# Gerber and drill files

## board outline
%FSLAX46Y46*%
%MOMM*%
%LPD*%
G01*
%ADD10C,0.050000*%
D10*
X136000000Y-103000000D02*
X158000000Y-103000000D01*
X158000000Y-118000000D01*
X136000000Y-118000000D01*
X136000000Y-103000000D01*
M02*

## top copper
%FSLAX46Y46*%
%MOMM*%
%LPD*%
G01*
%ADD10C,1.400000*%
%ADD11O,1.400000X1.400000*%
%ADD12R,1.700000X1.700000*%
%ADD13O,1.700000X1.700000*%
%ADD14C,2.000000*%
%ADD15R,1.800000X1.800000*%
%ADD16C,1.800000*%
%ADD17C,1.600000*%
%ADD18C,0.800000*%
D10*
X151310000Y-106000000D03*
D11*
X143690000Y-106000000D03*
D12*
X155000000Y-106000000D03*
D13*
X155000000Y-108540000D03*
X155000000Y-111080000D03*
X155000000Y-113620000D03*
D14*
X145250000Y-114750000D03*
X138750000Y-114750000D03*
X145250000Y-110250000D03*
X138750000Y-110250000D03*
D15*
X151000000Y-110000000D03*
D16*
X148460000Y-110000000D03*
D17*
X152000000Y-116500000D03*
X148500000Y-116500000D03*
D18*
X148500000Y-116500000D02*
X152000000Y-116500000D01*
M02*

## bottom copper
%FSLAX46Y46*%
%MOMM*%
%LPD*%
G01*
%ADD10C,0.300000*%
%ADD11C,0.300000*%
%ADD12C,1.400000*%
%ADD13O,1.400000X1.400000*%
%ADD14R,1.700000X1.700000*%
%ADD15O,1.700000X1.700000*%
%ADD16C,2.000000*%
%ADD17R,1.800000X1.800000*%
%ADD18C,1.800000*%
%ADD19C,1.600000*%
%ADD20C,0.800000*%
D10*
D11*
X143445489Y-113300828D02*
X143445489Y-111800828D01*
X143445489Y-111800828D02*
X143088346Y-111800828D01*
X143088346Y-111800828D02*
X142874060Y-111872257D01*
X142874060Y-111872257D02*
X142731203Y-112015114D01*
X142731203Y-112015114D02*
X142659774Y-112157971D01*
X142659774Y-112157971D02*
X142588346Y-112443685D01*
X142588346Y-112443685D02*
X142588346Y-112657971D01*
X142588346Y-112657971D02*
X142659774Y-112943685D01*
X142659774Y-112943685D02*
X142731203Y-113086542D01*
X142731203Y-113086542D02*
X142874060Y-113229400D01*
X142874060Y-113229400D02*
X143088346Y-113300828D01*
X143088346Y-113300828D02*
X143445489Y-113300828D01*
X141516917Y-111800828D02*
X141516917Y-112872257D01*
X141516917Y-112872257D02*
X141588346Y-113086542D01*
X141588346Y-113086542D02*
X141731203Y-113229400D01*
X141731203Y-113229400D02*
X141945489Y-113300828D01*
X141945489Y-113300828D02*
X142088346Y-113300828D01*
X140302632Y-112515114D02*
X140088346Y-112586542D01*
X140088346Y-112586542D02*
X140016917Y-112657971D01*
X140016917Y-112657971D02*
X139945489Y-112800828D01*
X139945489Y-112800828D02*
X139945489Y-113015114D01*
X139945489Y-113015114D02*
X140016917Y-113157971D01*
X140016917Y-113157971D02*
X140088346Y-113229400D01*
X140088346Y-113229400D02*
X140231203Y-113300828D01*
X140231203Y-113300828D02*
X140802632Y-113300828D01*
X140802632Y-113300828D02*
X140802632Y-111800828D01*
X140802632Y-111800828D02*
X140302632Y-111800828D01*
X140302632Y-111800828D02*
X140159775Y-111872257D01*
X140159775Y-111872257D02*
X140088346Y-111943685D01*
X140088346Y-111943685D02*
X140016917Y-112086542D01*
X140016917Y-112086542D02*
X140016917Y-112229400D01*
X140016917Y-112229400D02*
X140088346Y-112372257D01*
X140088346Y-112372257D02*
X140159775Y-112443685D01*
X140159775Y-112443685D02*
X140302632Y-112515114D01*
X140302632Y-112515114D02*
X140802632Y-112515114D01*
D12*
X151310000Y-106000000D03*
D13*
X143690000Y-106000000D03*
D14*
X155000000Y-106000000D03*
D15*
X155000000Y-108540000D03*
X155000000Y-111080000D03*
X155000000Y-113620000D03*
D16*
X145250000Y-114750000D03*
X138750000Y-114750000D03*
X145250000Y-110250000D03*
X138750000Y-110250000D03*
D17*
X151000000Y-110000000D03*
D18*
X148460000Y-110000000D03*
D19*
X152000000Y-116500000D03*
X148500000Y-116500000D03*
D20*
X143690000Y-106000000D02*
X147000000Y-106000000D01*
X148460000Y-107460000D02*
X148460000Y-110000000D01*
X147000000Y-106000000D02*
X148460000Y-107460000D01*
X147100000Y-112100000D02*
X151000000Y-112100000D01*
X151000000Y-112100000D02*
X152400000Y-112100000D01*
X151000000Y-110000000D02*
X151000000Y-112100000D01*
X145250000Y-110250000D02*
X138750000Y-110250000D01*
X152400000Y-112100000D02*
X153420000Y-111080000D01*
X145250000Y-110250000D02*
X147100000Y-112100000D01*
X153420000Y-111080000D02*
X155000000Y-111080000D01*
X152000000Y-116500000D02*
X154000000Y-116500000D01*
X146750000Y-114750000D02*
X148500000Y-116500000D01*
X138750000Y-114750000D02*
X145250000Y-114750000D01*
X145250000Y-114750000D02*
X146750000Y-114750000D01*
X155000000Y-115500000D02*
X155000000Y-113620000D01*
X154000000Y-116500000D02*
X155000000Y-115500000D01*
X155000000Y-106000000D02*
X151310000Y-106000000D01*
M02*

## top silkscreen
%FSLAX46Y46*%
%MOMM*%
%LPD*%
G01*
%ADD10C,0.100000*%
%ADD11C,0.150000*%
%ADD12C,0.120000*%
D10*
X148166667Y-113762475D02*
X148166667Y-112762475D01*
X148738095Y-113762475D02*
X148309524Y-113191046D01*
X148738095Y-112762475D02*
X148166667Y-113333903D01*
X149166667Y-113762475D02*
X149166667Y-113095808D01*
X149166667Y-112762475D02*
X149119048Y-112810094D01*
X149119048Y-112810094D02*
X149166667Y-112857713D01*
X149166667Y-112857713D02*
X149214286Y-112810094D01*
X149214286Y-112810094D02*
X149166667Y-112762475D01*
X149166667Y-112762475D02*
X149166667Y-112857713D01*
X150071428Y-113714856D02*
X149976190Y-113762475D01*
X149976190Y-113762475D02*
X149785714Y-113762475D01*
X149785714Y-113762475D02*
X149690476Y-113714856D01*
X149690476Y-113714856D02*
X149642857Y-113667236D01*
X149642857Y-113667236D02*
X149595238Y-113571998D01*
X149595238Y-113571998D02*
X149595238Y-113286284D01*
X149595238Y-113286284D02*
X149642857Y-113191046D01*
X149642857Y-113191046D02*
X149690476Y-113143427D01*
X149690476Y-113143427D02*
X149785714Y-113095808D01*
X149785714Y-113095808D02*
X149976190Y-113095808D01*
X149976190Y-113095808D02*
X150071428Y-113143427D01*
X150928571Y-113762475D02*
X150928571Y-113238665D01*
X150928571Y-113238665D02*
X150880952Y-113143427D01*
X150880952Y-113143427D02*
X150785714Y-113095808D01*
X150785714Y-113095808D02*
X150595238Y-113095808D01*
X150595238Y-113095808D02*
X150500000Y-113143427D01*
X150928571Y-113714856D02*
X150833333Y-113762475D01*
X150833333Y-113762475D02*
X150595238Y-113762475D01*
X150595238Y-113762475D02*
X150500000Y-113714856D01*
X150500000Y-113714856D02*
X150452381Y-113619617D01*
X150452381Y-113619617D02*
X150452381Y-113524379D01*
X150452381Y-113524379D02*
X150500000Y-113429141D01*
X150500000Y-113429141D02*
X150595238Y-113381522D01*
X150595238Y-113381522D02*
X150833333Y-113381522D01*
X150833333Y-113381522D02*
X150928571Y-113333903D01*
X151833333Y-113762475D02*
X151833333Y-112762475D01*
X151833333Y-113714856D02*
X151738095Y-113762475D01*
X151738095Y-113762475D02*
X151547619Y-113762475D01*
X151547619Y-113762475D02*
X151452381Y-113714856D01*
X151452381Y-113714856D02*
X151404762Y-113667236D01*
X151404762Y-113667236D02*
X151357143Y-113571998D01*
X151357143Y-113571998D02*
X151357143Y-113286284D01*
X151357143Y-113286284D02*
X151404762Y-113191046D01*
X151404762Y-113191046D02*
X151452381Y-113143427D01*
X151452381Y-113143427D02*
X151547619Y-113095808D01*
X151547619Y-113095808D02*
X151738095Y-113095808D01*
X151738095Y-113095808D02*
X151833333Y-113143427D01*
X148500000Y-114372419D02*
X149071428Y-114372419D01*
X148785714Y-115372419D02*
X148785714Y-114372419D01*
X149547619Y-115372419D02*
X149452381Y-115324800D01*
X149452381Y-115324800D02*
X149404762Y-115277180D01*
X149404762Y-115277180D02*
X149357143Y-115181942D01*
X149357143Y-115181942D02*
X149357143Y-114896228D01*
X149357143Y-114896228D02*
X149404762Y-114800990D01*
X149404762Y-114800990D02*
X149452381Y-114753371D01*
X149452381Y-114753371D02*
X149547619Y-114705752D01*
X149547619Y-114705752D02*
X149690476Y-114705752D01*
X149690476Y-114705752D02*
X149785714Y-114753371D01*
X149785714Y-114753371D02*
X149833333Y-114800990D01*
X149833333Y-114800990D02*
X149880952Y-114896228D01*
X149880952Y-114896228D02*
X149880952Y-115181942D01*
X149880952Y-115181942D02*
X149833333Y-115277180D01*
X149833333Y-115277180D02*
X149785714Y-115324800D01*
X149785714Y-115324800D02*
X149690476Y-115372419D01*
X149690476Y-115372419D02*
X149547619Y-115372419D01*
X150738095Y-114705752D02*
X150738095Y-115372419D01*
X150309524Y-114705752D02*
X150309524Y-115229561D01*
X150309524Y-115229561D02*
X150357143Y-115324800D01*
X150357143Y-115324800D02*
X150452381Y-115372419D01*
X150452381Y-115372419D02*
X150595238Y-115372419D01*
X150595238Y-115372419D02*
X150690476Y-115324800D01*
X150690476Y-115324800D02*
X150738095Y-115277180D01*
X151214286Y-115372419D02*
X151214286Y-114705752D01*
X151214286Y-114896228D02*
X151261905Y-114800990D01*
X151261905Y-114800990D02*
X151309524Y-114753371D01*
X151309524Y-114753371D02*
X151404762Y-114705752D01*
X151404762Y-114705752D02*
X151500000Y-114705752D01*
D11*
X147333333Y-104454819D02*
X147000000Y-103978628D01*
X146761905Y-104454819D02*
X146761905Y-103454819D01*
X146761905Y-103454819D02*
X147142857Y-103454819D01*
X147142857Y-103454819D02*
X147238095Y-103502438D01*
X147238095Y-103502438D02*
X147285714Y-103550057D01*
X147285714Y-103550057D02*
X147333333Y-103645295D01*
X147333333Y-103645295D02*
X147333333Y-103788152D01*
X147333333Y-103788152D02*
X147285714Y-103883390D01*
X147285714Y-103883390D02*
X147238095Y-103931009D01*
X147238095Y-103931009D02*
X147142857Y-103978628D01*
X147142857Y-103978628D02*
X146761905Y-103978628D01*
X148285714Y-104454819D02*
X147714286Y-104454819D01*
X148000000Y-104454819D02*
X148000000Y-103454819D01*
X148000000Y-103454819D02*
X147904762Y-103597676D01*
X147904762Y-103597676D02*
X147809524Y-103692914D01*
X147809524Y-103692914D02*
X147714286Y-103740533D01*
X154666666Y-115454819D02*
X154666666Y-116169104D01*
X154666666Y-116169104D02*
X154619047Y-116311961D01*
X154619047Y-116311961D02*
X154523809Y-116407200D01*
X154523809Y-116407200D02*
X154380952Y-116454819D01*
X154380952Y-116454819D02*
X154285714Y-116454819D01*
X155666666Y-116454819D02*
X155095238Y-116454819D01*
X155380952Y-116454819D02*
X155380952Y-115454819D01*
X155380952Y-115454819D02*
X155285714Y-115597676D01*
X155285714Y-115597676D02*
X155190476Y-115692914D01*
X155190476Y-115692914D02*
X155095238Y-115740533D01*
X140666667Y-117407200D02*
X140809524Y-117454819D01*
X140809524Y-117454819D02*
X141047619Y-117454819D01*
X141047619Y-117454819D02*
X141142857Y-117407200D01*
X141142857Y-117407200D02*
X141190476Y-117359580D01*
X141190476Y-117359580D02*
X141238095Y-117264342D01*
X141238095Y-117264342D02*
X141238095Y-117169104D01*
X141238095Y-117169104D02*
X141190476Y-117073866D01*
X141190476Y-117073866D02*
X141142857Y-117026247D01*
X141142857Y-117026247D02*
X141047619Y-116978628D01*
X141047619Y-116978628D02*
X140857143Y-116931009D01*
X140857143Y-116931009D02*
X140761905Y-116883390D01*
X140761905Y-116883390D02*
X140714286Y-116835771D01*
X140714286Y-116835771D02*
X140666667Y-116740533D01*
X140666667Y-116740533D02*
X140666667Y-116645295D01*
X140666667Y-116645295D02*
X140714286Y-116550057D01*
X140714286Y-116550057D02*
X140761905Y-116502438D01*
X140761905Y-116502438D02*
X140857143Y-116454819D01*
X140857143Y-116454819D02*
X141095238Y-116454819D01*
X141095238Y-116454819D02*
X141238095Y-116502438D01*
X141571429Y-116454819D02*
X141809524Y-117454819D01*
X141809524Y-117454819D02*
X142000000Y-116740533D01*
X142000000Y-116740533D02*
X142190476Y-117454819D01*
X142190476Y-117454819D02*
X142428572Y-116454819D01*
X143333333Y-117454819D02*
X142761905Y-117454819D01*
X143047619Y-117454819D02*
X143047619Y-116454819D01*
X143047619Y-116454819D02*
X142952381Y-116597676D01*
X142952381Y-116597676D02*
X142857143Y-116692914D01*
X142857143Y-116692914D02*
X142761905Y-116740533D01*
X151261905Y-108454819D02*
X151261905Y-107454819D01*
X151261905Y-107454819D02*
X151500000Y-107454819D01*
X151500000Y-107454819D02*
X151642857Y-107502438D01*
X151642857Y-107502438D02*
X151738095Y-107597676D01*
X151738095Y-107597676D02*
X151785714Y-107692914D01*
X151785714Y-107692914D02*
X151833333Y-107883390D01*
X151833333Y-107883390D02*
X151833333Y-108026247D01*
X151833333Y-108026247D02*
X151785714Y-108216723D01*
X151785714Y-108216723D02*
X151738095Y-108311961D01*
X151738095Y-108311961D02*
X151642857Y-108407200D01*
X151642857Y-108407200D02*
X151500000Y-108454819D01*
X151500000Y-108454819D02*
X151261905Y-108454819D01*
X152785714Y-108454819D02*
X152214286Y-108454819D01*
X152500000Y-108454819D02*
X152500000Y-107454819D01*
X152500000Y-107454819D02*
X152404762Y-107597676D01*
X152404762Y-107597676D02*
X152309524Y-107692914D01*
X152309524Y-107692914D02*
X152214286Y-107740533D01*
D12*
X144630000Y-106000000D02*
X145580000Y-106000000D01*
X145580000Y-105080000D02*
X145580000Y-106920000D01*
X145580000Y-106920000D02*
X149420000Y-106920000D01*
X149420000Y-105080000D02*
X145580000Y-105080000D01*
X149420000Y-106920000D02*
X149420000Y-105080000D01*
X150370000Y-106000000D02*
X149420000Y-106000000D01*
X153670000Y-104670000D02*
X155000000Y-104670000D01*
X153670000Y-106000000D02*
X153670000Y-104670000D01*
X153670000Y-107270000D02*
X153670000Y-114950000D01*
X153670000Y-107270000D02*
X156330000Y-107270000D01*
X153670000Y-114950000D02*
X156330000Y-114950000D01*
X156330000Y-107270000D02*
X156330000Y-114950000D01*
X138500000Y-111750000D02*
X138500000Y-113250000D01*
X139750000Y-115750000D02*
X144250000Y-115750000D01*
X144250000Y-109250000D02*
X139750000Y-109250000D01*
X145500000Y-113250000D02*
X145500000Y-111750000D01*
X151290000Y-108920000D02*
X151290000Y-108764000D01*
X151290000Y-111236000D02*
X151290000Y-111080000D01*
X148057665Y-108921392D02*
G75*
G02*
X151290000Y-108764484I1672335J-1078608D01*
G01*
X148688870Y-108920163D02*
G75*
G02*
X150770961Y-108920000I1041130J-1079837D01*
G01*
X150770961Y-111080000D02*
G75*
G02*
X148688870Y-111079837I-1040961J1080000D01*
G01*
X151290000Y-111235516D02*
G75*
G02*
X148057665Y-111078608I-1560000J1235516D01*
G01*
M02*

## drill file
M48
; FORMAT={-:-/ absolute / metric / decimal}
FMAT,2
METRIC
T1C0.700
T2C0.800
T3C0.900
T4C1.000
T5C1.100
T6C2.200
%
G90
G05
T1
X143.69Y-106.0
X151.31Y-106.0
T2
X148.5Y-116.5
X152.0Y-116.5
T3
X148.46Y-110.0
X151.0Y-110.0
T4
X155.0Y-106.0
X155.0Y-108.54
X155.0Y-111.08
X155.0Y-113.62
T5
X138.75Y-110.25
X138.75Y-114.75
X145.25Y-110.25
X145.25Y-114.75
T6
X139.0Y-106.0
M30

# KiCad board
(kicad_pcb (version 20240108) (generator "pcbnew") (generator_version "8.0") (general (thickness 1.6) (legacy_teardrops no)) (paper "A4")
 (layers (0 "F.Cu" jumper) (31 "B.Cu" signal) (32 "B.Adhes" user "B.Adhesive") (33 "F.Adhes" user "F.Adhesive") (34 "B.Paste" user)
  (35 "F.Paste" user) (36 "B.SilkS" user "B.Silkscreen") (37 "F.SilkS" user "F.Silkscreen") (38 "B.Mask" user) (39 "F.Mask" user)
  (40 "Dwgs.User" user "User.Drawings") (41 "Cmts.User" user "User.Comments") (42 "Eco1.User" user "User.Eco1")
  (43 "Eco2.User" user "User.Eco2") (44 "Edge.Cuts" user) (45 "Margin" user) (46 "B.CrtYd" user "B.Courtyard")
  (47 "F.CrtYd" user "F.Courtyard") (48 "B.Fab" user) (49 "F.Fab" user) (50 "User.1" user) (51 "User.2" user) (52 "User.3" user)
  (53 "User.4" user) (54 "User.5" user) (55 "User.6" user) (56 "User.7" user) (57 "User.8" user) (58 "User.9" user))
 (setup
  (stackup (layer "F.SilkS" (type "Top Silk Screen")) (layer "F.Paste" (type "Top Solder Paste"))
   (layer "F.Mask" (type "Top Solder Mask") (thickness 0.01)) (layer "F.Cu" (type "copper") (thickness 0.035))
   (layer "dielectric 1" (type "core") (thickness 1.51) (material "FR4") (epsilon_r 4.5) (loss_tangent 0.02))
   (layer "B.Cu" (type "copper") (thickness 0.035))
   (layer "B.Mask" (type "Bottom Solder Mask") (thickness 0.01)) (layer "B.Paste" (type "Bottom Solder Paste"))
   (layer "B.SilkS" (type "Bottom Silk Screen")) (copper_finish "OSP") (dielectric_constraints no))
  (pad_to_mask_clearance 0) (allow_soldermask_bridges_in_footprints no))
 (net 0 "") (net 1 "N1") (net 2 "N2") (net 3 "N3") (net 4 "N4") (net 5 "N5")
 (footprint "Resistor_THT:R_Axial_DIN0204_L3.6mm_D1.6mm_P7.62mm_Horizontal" (layer "F.Cu") (at 151.31 106 180)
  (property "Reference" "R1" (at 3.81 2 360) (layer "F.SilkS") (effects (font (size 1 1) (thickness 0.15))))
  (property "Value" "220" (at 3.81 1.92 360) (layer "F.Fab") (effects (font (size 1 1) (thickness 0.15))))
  (fp_line (start 6.68 0) (end 5.73 0) (stroke (width 0.12) (type solid)) (layer "F.SilkS"))
  (fp_line (start 5.73 0.92) (end 5.73 -0.92) (stroke (width 0.12) (type solid)) (layer "F.SilkS"))
  (fp_line (start 5.73 -0.92) (end 1.89 -0.92) (stroke (width 0.12) (type solid)) (layer "F.SilkS"))
  (fp_line (start 1.89 0.92) (end 5.73 0.92) (stroke (width 0.12) (type solid)) (layer "F.SilkS"))
  (fp_line (start 1.89 -0.92) (end 1.89 0.92) (stroke (width 0.12) (type solid)) (layer "F.SilkS"))
  (fp_line (start 0.94 0) (end 1.89 0) (stroke (width 0.12) (type solid)) (layer "F.SilkS"))
  (pad "1" thru_hole circle (at 0 0 180) (size 1.4 1.4) (drill 0.7) (layers "*.Cu" "*.Mask") (remove_unused_layers no) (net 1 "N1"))
  (pad "2" thru_hole oval (at 7.62 0 180) (size 1.4 1.4) (drill 0.7) (layers "*.Cu" "*.Mask") (remove_unused_layers no) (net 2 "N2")))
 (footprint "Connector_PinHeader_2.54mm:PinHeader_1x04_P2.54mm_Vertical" (layer "F.Cu") (at 155 106)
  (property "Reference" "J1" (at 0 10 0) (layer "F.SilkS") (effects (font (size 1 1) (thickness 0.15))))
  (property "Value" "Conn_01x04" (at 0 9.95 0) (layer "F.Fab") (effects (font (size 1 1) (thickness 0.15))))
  (fp_line (start -1.33 -1.33) (end 0 -1.33) (stroke (width 0.12) (type solid)) (layer "F.SilkS"))
  (fp_line (start -1.33 0) (end -1.33 -1.33) (stroke (width 0.12) (type solid)) (layer "F.SilkS"))
  (fp_line (start -1.33 1.27) (end -1.33 8.95) (stroke (width 0.12) (type solid)) (layer "F.SilkS"))
  (fp_line (start -1.33 1.27) (end 1.33 1.27) (stroke (width 0.12) (type solid)) (layer "F.SilkS"))
  (fp_line (start -1.33 8.95) (end 1.33 8.95) (stroke (width 0.12) (type solid)) (layer "F.SilkS"))
  (fp_line (start 1.33 1.27) (end 1.33 8.95) (stroke (width 0.12) (type solid)) (layer "F.SilkS"))
  (pad "1" thru_hole rect (at 0 0) (size 1.7 1.7) (drill 1) (layers "*.Cu" "*.Mask") (remove_unused_layers no) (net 1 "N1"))
  (pad "2" thru_hole oval (at 0 2.54) (size 1.7 1.7) (drill 1) (layers "*.Cu" "*.Mask") (remove_unused_layers no) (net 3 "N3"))
  (pad "3" thru_hole oval (at 0 5.08) (size 1.7 1.7) (drill 1) (layers "*.Cu" "*.Mask") (remove_unused_layers no) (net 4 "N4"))
  (pad "4" thru_hole oval (at 0 7.62) (size 1.7 1.7) (drill 1) (layers "*.Cu" "*.Mask") (remove_unused_layers no) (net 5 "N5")))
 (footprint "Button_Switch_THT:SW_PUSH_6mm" (layer "F.Cu") (at 145.25 114.75 180)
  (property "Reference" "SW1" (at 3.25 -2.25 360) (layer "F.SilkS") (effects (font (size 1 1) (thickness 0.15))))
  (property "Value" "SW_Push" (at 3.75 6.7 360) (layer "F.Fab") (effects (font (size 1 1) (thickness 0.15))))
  (fp_line (start 6.75 3) (end 6.75 1.5) (stroke (width 0.12) (type solid)) (layer "F.SilkS"))
  (fp_line (start 5.5 -1) (end 1 -1) (stroke (width 0.12) (type solid)) (layer "F.SilkS"))
  (fp_line (start 1 5.5) (end 5.5 5.5) (stroke (width 0.12) (type solid)) (layer "F.SilkS"))
  (fp_line (start -0.25 1.5) (end -0.25 3) (stroke (width 0.12) (type solid)) (layer "F.SilkS"))
  (pad "1" thru_hole circle (at 0 0 270) (size 2 2) (drill 1.1) (layers "*.Cu" "*.Mask") (remove_unused_layers no) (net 5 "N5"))
  (pad "1" thru_hole circle (at 6.5 0 270) (size 2 2) (drill 1.1) (layers "*.Cu" "*.Mask") (remove_unused_layers no) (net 5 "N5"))
  (pad "2" thru_hole circle (at 0 4.5 270) (size 2 2) (drill 1.1) (layers "*.Cu" "*.Mask") (remove_unused_layers no) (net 4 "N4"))
  (pad "2" thru_hole circle (at 6.5 4.5 270) (size 2 2) (drill 1.1) (layers "*.Cu" "*.Mask") (remove_unused_layers no) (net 4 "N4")))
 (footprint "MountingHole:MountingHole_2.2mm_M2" (layer "F.Cu") (at 139 106)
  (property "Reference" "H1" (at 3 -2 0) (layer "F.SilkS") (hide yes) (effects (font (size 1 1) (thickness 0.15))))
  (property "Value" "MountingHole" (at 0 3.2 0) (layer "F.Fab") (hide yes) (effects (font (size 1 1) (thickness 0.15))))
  (pad "" np_thru_hole circle (at 0 0) (size 2.2 2.2) (drill 2.2) (layers "*.Cu" "*.Mask")))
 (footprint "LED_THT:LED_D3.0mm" (layer "F.Cu") (at 151 110 180)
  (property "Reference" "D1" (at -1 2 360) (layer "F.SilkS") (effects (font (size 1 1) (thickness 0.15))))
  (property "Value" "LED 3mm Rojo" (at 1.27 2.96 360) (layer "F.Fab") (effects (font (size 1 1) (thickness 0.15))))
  (fp_line (start -0.29 1.08) (end -0.29 1.236) (stroke (width 0.12) (type solid)) (layer "F.SilkS"))
  (fp_line (start -0.29 -1.236) (end -0.29 -1.08) (stroke (width 0.12) (type solid)) (layer "F.SilkS"))
  (fp_arc (start 2.942335 1.078608) (mid 1.366487 1.987659) (end -0.29 1.235516) (stroke (width 0.12) (type solid)) (layer "F.SilkS"))
  (fp_arc (start 2.31113 1.079837) (mid 1.270117 1.5) (end 0.229039 1.08) (stroke (width 0.12) (type solid)) (layer "F.SilkS"))
  (fp_arc (start 0.229039 -1.08) (mid 1.270117 -1.5) (end 2.31113 -1.079837) (stroke (width 0.12) (type solid)) (layer "F.SilkS"))
  (fp_arc (start -0.29 -1.235516) (mid 1.366487 -1.987659) (end 2.942335 -1.078608) (stroke (width 0.12) (type solid)) (layer "F.SilkS"))
  (pad "1" thru_hole rect (at 0 0 180) (size 1.8 1.8) (drill 0.9) (layers "*.Cu" "*.Mask") (remove_unused_layers no) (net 4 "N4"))
  (pad "2" thru_hole circle (at 2.54 0 180) (size 1.8 1.8) (drill 0.9) (layers "*.Cu" "*.Mask") (remove_unused_layers no) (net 2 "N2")))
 (gr_rect (start 136 103) (end 158 118) (stroke (width 0.05) (type default)) (fill none) (layer "Edge.Cuts"))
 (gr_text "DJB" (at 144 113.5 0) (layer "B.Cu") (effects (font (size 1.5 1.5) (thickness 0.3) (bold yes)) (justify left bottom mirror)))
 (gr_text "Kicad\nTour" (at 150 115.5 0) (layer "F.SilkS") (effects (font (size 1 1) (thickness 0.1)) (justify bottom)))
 (segment (start 143.69 106) (end 147 106) (width 0.8) (layer "B.Cu") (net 2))
 (segment (start 148.46 107.46) (end 148.46 110) (width 0.8) (layer "B.Cu") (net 2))
 (segment (start 147 106) (end 148.46 107.46) (width 0.8) (layer "B.Cu") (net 2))
 (segment (start 147.1 112.1) (end 151 112.1) (width 0.8) (layer "B.Cu") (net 4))
 (segment (start 151 112.1) (end 152.4 112.1) (width 0.8) (layer "B.Cu") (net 4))
 (segment (start 151 110) (end 151 112.1) (width 0.8) (layer "B.Cu") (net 4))
 (segment (start 145.25 110.25) (end 138.75 110.25) (width 0.8) (layer "B.Cu") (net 4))
 (segment (start 152.4 112.1) (end 153.42 111.08) (width 0.8) (layer "B.Cu") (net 4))
 (segment (start 145.25 110.25) (end 147.1 112.1) (width 0.8) (layer "B.Cu") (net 4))
 (segment (start 153.42 111.08) (end 155 111.08) (width 0.8) (layer "B.Cu") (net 4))
 (segment (start 148.5 116.5) (end 152 116.5) (width 0.8) (layer "F.Cu") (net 5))
 (via (at 152 116.5) (size 1.6) (drill 0.8) (layers "F.Cu" "B.Cu") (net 5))
 (via (at 148.5 116.5) (size 1.6) (drill 0.8) (layers "F.Cu" "B.Cu") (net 5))
 (segment (start 152 116.5) (end 154 116.5) (width 0.8) (layer "B.Cu") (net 5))
 (segment (start 146.75 114.75) (end 148.5 116.5) (width 0.8) (layer "B.Cu") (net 5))
 (segment (start 138.75 114.75) (end 145.25 114.75) (width 0.8) (layer "B.Cu") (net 5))
 (segment (start 145.25 114.75) (end 146.75 114.75) (width 0.8) (layer "B.Cu") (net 5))
 (segment (start 155 115.5) (end 155 113.62) (width 0.8) (layer "B.Cu") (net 5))
 (segment (start 154 116.5) (end 155 115.5) (width 0.8) (layer "B.Cu") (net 5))
 (segment (start 155 106) (end 151.31 106) (width 0.8) (layer "B.Cu") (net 1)))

